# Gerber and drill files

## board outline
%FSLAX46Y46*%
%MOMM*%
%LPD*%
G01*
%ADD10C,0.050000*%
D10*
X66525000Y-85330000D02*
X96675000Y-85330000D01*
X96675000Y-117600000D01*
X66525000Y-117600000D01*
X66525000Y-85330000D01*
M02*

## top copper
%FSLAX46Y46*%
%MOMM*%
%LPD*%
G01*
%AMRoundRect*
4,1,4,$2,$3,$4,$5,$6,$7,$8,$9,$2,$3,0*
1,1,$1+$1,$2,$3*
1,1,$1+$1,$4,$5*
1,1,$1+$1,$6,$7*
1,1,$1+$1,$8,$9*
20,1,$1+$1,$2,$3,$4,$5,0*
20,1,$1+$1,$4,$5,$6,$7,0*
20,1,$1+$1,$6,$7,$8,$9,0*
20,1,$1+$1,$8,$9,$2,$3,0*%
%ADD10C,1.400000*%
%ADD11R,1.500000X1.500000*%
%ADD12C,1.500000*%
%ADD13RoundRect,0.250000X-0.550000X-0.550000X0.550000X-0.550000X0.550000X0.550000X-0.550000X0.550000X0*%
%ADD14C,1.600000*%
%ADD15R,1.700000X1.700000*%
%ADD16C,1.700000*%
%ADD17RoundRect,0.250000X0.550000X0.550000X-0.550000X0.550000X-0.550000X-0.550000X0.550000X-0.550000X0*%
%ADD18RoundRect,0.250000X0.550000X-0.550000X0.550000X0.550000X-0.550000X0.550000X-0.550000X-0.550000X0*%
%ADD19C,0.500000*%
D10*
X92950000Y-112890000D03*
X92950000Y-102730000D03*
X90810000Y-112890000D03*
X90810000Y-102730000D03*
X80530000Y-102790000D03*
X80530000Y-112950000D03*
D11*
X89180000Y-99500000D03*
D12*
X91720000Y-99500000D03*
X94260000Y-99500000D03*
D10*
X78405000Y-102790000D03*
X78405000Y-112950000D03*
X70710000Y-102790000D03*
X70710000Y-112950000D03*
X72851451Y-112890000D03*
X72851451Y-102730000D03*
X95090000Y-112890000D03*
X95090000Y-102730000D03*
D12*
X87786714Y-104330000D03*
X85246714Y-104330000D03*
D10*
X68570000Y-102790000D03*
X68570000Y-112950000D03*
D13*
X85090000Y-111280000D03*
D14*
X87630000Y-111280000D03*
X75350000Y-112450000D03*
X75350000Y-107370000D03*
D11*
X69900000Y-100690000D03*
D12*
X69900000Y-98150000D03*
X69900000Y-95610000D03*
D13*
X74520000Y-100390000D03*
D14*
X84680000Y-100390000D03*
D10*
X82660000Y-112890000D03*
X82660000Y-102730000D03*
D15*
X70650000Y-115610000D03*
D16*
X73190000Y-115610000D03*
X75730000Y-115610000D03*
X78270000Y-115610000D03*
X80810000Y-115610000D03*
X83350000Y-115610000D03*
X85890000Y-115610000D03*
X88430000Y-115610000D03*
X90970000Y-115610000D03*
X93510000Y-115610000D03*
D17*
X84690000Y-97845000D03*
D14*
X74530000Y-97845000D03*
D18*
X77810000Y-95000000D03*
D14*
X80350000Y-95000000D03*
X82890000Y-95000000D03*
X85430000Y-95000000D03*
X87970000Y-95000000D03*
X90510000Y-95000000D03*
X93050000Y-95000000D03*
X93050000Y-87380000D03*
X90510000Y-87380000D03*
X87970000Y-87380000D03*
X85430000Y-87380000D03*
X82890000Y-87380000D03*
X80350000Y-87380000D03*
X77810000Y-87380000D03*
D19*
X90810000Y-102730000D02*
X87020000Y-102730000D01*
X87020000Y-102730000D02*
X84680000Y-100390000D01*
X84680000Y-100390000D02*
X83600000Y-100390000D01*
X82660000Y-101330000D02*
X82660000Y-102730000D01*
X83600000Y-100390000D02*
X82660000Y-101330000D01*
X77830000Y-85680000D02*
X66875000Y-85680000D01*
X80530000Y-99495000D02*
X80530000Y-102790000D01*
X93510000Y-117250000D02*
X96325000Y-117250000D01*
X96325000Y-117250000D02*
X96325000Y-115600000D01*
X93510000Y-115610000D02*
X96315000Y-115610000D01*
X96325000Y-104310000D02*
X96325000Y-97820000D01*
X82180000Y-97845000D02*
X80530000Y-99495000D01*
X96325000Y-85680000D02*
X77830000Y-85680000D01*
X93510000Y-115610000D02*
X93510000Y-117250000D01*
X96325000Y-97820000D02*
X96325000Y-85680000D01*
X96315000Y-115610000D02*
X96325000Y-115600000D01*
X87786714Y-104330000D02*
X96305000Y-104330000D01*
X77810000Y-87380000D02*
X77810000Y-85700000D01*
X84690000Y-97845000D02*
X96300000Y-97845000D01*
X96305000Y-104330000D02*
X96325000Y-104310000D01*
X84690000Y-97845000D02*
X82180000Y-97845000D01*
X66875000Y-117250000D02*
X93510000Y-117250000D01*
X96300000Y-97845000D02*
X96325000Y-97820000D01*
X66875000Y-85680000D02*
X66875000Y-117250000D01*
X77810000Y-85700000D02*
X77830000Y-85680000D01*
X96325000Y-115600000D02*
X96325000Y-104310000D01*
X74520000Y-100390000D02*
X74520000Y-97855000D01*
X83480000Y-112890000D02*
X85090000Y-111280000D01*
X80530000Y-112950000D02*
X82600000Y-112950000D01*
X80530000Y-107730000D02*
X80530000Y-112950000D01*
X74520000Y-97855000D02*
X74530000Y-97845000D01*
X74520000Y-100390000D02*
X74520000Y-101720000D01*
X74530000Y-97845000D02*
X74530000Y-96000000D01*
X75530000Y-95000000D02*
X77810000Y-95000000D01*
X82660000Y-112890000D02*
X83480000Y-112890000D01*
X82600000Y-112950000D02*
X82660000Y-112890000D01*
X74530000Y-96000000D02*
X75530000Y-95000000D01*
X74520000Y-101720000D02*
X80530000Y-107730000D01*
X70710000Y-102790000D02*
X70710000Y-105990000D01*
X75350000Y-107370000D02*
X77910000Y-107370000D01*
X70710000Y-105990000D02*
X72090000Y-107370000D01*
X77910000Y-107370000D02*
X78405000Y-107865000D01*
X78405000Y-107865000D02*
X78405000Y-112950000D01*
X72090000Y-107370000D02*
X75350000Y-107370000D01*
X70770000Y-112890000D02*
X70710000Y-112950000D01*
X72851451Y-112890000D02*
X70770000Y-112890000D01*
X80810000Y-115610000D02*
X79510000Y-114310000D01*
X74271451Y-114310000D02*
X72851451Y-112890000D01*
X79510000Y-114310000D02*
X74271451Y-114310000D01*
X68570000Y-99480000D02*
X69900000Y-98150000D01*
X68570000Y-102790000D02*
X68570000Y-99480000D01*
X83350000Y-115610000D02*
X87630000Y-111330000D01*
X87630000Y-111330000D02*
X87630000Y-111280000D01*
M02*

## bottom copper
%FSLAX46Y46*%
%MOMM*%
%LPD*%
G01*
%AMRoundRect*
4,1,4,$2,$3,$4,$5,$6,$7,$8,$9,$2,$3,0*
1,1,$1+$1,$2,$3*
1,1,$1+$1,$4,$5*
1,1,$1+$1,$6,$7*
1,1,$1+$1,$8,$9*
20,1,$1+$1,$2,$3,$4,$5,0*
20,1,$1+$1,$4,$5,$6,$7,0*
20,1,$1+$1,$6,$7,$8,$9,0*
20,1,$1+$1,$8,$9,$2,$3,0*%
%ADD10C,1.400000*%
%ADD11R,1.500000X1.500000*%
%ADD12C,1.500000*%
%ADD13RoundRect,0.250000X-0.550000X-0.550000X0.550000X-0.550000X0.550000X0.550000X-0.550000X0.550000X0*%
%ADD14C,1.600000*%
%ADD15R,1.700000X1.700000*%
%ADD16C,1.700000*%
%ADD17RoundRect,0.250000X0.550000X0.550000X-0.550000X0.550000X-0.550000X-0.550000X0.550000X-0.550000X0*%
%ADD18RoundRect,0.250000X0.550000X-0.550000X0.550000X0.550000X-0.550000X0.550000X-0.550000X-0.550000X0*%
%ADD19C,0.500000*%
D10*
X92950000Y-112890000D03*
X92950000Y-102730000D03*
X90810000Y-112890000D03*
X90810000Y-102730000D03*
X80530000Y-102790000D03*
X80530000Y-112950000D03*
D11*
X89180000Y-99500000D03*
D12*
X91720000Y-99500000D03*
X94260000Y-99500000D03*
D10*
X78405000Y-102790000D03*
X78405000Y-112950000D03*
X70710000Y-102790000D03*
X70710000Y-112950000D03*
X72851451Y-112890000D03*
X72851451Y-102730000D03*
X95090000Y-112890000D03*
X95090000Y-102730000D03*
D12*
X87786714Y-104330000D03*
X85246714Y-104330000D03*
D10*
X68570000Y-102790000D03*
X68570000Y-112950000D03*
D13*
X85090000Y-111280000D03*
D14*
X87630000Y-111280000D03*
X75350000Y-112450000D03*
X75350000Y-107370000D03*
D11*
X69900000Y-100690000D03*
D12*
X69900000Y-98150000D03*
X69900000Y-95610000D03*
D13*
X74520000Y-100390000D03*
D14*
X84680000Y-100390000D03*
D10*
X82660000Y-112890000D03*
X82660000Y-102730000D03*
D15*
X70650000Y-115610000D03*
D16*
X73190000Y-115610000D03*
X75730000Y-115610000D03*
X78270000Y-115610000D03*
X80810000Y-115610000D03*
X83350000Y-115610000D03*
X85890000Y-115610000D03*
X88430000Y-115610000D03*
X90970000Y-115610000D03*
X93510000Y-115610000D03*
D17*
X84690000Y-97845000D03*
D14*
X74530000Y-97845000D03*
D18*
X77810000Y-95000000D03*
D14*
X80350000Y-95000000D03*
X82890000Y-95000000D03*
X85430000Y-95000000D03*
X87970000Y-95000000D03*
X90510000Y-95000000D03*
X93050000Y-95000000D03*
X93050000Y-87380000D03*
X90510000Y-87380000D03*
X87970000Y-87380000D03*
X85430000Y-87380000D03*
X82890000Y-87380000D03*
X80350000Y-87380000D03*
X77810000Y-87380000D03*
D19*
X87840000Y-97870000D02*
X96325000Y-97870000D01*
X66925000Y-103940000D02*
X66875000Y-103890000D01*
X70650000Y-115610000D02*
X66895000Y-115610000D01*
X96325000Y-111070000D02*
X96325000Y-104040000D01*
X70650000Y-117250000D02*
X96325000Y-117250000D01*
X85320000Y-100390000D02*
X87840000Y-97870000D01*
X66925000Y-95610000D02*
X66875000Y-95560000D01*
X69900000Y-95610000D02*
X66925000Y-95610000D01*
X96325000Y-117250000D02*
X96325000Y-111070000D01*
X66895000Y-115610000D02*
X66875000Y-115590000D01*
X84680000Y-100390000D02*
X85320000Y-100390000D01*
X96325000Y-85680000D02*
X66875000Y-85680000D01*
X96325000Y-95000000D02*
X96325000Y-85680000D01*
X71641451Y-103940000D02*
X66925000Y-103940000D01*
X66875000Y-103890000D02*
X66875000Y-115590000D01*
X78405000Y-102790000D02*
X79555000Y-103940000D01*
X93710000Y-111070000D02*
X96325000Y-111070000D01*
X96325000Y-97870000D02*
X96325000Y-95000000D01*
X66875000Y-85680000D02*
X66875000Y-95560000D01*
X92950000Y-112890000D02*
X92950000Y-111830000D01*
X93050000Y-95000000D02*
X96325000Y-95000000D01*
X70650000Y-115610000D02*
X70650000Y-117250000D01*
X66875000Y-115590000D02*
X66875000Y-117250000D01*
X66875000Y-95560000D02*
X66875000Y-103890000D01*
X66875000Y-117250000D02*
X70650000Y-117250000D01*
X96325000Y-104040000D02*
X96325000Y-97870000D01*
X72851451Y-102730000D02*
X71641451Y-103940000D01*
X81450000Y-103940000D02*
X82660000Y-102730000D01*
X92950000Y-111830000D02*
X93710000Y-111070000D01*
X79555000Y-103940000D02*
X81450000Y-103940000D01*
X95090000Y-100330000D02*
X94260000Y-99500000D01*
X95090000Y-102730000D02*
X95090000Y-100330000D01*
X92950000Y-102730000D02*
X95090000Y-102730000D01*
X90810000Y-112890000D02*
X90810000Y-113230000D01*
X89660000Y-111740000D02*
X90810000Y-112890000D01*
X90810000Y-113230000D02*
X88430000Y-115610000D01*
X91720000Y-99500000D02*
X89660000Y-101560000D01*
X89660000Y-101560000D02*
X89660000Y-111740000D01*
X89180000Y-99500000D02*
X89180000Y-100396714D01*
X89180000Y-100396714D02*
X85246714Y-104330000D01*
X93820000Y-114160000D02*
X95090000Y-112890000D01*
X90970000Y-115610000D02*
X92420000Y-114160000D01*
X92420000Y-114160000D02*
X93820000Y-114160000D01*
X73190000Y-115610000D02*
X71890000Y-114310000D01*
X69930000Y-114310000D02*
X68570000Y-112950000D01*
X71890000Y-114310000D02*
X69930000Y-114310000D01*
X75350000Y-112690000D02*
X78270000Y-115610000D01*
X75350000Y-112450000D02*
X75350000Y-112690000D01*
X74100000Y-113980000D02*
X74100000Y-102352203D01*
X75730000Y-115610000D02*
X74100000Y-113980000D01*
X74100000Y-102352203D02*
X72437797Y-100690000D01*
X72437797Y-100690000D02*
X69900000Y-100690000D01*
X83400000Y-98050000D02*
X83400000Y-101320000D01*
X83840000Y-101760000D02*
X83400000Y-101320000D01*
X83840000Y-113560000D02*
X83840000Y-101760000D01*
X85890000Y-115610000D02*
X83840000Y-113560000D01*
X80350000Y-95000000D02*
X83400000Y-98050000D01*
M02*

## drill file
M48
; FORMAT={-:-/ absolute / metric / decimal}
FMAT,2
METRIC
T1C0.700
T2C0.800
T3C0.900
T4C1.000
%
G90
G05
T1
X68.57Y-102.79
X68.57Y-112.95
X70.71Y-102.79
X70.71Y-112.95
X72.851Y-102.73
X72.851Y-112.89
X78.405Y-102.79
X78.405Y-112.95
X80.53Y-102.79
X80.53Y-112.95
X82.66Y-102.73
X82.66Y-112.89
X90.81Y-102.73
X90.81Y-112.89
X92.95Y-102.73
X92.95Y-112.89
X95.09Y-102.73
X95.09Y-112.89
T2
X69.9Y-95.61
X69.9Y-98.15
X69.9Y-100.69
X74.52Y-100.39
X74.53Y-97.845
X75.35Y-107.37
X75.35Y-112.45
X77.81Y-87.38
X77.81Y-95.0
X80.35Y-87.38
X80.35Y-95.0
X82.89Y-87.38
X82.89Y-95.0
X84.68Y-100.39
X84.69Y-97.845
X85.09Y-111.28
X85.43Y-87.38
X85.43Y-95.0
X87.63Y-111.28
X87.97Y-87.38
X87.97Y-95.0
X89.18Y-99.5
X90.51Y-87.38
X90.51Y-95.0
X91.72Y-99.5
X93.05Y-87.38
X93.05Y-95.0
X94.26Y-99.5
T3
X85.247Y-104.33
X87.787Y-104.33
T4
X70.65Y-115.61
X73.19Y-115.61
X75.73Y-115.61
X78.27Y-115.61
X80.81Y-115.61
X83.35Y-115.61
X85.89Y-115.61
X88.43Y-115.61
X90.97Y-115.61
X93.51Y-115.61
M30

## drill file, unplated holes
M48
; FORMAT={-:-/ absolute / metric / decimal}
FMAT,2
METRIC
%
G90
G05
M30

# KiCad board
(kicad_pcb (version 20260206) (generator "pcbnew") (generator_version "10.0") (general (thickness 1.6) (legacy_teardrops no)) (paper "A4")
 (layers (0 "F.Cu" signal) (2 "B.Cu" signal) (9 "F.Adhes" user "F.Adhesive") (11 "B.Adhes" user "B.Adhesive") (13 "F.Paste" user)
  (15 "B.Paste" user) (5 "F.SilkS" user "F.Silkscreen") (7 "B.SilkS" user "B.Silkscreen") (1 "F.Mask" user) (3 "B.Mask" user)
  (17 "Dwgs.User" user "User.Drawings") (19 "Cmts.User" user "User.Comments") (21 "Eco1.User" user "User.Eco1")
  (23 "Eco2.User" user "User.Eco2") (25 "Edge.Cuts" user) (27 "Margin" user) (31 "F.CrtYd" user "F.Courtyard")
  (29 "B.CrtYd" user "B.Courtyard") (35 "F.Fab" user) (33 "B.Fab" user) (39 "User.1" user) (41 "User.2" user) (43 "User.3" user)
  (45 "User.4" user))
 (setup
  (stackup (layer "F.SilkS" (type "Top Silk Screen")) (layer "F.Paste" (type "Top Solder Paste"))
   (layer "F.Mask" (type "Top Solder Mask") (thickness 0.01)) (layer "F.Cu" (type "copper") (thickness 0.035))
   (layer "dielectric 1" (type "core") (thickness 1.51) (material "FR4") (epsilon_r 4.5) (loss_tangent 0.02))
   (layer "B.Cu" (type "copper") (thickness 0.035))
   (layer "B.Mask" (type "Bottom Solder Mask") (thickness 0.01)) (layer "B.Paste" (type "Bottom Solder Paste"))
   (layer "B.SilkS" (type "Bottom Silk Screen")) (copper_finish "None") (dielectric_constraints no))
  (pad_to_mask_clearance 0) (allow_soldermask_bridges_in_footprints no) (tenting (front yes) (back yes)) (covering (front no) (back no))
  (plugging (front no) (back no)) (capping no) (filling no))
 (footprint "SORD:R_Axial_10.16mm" (layer "F.Cu") (at 92.95 112.89 90)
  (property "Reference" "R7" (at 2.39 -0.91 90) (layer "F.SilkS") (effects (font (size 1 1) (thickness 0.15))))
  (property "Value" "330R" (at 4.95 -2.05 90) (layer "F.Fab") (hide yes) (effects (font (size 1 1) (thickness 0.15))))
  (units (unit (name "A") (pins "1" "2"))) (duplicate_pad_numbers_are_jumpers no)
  (pad "1" thru_hole circle (at 0 0 90) (size 1.4 1.4) (drill 0.7) (layers "*.Cu" "*.Mask") (remove_unused_layers no) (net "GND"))
  (pad "2" thru_hole circle (at 10.16 0 90) (size 1.4 1.4) (drill 0.7) (layers "*.Cu" "*.Mask") (remove_unused_layers no) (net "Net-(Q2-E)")))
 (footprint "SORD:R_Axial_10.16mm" (layer "F.Cu") (at 90.81 112.89 90)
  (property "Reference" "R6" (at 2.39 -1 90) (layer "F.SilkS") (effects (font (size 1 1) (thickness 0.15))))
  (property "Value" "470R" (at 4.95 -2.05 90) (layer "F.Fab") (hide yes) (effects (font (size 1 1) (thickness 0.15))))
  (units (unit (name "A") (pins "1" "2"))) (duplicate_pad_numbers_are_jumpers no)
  (pad "1" thru_hole circle (at 0 0 90) (size 1.4 1.4) (drill 0.7) (layers "*.Cu" "*.Mask") (remove_unused_layers no) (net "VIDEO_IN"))
  (pad "2" thru_hole circle (at 10.16 0 90) (size 1.4 1.4) (drill 0.7) (layers "*.Cu" "*.Mask") (remove_unused_layers no) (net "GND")))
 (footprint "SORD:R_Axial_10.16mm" (layer "F.Cu") (at 80.53 102.79 -90)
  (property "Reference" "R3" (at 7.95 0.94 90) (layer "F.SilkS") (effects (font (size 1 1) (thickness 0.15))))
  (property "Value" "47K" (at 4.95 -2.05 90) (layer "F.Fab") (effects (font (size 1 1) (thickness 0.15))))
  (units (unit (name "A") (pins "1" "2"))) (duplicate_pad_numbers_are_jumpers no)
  (pad "1" thru_hole circle (at 0 0 270) (size 1.4 1.4) (drill 0.7) (layers "*.Cu" "*.Mask") (remove_unused_layers no) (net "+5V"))
  (pad "2" thru_hole circle (at 10.16 0 270) (size 1.4 1.4) (drill 0.7) (layers "*.Cu" "*.Mask") (remove_unused_layers no)
   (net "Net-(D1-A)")))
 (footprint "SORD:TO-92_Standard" (layer "F.Cu") (at 89.18 99.5)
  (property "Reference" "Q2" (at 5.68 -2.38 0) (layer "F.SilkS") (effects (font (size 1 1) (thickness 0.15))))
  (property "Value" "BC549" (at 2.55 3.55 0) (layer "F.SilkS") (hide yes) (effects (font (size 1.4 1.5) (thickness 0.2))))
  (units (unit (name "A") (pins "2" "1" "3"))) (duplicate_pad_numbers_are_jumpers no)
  (pad "1" thru_hole rect (at 0 0) (size 1.5 1.5) (drill 0.8) (layers "*.Cu" "*.Mask") (remove_unused_layers no) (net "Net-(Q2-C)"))
  (pad "2" thru_hole circle (at 2.54 0) (size 1.5 1.5) (drill 0.8) (layers "*.Cu" "*.Mask") (remove_unused_layers no) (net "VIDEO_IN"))
  (pad "3" thru_hole circle (at 5.08 0) (size 1.5 1.5) (drill 0.8) (layers "*.Cu" "*.Mask") (remove_unused_layers no) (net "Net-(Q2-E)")))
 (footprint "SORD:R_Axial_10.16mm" (layer "F.Cu") (at 78.405 102.79 -90)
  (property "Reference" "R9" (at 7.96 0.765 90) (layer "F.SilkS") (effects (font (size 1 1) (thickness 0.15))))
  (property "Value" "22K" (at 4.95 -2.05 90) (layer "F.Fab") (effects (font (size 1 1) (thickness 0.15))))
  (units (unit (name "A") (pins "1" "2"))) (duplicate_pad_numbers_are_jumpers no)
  (pad "1" thru_hole circle (at 0 0 270) (size 1.4 1.4) (drill 0.7) (layers "*.Cu" "*.Mask") (remove_unused_layers no) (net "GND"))
  (pad "2" thru_hole circle (at 10.16 0 270) (size 1.4 1.4) (drill 0.7) (layers "*.Cu" "*.Mask") (remove_unused_layers no)
   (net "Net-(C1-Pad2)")))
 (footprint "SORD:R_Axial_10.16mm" (layer "F.Cu") (at 70.71 102.79 -90)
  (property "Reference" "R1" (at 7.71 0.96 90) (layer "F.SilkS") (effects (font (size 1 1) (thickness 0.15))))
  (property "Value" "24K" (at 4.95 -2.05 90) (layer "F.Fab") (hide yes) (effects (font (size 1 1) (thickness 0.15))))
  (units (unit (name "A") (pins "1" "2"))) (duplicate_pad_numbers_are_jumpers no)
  (pad "1" thru_hole circle (at 0 0 270) (size 1.4 1.4) (drill 0.7) (layers "*.Cu" "*.Mask") (remove_unused_layers no) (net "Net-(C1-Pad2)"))
  (pad "2" thru_hole circle (at 10.16 0 270) (size 1.4 1.4) (drill 0.7) (layers "*.Cu" "*.Mask") (remove_unused_layers no) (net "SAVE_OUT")))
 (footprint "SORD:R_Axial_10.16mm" (layer "F.Cu") (at 72.851451 112.89 90)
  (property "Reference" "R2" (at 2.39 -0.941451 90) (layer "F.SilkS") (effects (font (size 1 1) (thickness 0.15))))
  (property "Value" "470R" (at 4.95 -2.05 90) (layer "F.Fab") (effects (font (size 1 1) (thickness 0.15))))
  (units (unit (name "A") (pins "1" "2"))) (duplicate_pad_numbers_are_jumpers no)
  (pad "1" thru_hole circle (at 0 0 90) (size 1.4 1.4) (drill 0.7) (layers "*.Cu" "*.Mask") (remove_unused_layers no) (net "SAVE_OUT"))
  (pad "2" thru_hole circle (at 10.16 0 90) (size 1.4 1.4) (drill 0.7) (layers "*.Cu" "*.Mask") (remove_unused_layers no) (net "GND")))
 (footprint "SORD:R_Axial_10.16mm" (layer "F.Cu") (at 95.09 112.89 90)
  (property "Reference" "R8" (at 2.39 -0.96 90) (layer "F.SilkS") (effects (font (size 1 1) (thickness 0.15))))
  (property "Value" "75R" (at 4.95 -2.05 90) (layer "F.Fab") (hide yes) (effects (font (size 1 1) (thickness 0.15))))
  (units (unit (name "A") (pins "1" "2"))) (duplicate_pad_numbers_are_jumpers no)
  (pad "1" thru_hole circle (at 0 0 90) (size 1.4 1.4) (drill 0.7) (layers "*.Cu" "*.Mask") (remove_unused_layers no) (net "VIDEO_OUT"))
  (pad "2" thru_hole circle (at 10.16 0 90) (size 1.4 1.4) (drill 0.7) (layers "*.Cu" "*.Mask") (remove_unused_layers no) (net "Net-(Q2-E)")))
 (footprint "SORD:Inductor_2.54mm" (layer "F.Cu") (at 87.786714 104.33 180)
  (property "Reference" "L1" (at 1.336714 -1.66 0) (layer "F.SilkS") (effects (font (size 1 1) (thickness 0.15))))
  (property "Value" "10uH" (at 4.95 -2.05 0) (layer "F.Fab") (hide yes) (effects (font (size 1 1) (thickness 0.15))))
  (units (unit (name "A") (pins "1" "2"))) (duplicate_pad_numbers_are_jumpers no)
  (pad "1" thru_hole circle (at 0 0 180) (size 1.5 1.5) (drill 0.9) (layers "*.Cu" "*.Mask") (remove_unused_layers no) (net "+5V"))
  (pad "2" thru_hole circle (at 2.54 0 180) (size 1.5 1.5) (drill 0.9) (layers "*.Cu" "*.Mask") (remove_unused_layers no) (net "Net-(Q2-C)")))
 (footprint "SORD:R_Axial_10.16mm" (layer "F.Cu") (at 68.57 102.79 -90)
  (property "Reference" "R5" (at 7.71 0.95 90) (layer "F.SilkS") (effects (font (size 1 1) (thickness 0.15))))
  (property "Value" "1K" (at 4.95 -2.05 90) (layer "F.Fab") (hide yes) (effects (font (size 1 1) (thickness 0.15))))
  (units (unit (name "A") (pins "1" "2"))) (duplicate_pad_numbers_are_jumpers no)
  (pad "1" thru_hole circle (at 0 0 270) (size 1.4 1.4) (drill 0.7) (layers "*.Cu" "*.Mask") (remove_unused_layers no) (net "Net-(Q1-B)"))
  (pad "2" thru_hole circle (at 10.16 0 270) (size 1.4 1.4) (drill 0.7) (layers "*.Cu" "*.Mask") (remove_unused_layers no) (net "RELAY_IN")))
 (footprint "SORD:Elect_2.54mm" (layer "F.Cu") (at 85.09 111.28)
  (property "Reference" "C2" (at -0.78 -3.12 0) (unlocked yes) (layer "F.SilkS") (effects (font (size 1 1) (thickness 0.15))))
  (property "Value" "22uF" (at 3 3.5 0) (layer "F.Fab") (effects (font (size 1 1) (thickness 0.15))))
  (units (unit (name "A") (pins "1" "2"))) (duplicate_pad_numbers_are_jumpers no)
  (pad "1" thru_hole roundrect (at 0 0) (size 1.6 1.6) (drill 0.8) (layers "*.Cu" "*.Mask") (remove_unused_layers no)
   (roundrect_rratio 0.15625) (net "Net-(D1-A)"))
  (pad "2" thru_hole circle (at 2.54 0) (size 1.6 1.6) (drill 0.8) (layers "*.Cu" "*.Mask") (remove_unused_layers no) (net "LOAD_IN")))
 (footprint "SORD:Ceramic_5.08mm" (layer "F.Cu") (at 75.35 112.45 90)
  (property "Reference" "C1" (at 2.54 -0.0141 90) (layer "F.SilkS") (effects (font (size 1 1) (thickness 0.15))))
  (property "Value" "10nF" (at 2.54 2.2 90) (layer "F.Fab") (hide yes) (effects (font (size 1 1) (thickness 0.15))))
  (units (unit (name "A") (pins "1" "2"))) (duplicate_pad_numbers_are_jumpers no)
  (pad "1" thru_hole circle (at 0 0 90) (size 1.6 1.6) (drill 0.8) (layers "*.Cu" "*.Mask") (remove_unused_layers no) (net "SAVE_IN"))
  (pad "2" thru_hole circle (at 5.08 0 90) (size 1.6 1.6) (drill 0.8) (layers "*.Cu" "*.Mask") (remove_unused_layers no)
   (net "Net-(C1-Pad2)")))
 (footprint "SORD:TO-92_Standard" (layer "F.Cu") (at 69.9 100.69 90)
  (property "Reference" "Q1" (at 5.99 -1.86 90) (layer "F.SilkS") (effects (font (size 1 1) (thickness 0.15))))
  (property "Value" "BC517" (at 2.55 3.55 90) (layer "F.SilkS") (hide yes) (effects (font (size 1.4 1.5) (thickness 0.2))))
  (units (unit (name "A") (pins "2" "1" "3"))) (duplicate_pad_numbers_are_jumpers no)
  (pad "1" thru_hole rect (at 0 0 90) (size 1.5 1.5) (drill 0.8) (layers "*.Cu" "*.Mask") (remove_unused_layers no) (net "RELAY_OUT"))
  (pad "2" thru_hole circle (at 2.54 0 90) (size 1.5 1.5) (drill 0.8) (layers "*.Cu" "*.Mask") (remove_unused_layers no) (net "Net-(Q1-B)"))
  (pad "3" thru_hole circle (at 5.08 0 90) (size 1.5 1.5) (drill 0.8) (layers "*.Cu" "*.Mask") (remove_unused_layers no) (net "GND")))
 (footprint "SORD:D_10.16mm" (layer "F.Cu") (at 74.52 100.39)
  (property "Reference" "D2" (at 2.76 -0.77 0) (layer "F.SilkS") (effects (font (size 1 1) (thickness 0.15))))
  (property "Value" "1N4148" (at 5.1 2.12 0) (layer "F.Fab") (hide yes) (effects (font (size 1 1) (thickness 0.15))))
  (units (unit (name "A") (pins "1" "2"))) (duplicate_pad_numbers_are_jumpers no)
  (pad "1" thru_hole roundrect (at 0 0) (size 1.6 1.6) (drill 0.8) (layers "*.Cu" "*.Mask") (remove_unused_layers no)
   (roundrect_rratio 0.15625) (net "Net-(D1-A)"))
  (pad "2" thru_hole circle (at 10.16 0) (size 1.6 1.6) (drill 0.8) (layers "*.Cu" "*.Mask") (remove_unused_layers no) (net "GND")))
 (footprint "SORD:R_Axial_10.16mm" (layer "F.Cu") (at 82.66 112.89 90)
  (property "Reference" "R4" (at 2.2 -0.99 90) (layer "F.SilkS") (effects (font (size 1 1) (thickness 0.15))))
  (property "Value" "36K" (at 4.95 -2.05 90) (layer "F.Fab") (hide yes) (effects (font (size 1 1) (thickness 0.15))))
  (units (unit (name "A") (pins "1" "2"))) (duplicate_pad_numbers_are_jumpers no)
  (pad "1" thru_hole circle (at 0 0 90) (size 1.4 1.4) (drill 0.7) (layers "*.Cu" "*.Mask") (remove_unused_layers no) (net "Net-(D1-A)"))
  (pad "2" thru_hole circle (at 10.16 0 90) (size 1.4 1.4) (drill 0.7) (layers "*.Cu" "*.Mask") (remove_unused_layers no) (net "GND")))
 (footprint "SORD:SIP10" (layer "F.Cu") (at 70.65 115.61)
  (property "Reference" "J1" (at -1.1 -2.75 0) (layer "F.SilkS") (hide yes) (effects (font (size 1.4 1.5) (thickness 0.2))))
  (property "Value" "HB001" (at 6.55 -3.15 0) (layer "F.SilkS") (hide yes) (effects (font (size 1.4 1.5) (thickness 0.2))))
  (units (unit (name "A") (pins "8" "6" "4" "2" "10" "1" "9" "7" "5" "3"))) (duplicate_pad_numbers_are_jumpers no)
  (pad "1" thru_hole rect (at 0 0) (size 1.7 1.7) (drill 1) (layers "*.Cu" "*.Mask") (remove_unused_layers no) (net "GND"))
  (pad "2" thru_hole circle (at 2.54 0) (size 1.7 1.7) (drill 1) (layers "*.Cu" "*.Mask") (remove_unused_layers no) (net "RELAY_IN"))
  (pad "3" thru_hole circle (at 5.08 0) (size 1.7 1.7) (drill 1) (layers "*.Cu" "*.Mask") (remove_unused_layers no) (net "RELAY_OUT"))
  (pad "4" thru_hole circle (at 7.62 0) (size 1.7 1.7) (drill 1) (layers "*.Cu" "*.Mask") (remove_unused_layers no) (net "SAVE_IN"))
  (pad "5" thru_hole circle (at 10.16 0) (size 1.7 1.7) (drill 1) (layers "*.Cu" "*.Mask") (remove_unused_layers no) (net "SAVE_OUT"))
  (pad "6" thru_hole circle (at 12.7 0) (size 1.7 1.7) (drill 1) (layers "*.Cu" "*.Mask") (remove_unused_layers no) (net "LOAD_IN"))
  (pad "7" thru_hole circle (at 15.24 0) (size 1.7 1.7) (drill 1) (layers "*.Cu" "*.Mask") (remove_unused_layers no) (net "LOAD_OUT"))
  (pad "8" thru_hole circle (at 17.78 0) (size 1.7 1.7) (drill 1) (layers "*.Cu" "*.Mask") (remove_unused_layers no) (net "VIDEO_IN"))
  (pad "9" thru_hole circle (at 20.32 0) (size 1.7 1.7) (drill 1) (layers "*.Cu" "*.Mask") (remove_unused_layers no) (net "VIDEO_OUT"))
  (pad "10" thru_hole circle (at 22.86 0) (size 1.7 1.7) (drill 1) (layers "*.Cu" "*.Mask") (remove_unused_layers no) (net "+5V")))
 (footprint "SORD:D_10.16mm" (layer "F.Cu") (at 84.69 97.845 180)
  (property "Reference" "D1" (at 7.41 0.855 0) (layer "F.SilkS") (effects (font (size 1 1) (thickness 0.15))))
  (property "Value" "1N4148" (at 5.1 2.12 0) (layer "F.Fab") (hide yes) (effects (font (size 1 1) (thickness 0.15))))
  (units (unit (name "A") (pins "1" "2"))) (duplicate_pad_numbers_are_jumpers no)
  (pad "1" thru_hole roundrect (at 0 0 180) (size 1.6 1.6) (drill 0.8) (layers "*.Cu" "*.Mask") (remove_unused_layers no)
   (roundrect_rratio 0.15625) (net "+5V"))
  (pad "2" thru_hole circle (at 10.16 0 180) (size 1.6 1.6) (drill 0.8) (layers "*.Cu" "*.Mask") (remove_unused_layers no)
   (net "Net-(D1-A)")))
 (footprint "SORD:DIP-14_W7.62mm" (layer "F.Cu") (at 77.81 95 90)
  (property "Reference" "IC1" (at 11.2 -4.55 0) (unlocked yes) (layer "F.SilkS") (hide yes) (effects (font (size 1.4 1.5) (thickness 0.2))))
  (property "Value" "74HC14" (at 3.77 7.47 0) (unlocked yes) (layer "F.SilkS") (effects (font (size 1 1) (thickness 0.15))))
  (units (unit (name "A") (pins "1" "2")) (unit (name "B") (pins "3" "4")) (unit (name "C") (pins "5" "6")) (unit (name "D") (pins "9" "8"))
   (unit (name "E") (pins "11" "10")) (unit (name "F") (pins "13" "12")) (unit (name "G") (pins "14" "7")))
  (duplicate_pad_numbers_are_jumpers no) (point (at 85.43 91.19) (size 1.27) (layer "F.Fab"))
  (pad "1" thru_hole roundrect (at 0 0 90) (size 1.6 1.6) (drill 0.8) (layers "*.Cu" "*.Mask") (remove_unused_layers no)
   (roundrect_rratio 0.15625) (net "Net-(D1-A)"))
  (pad "2" thru_hole circle (at 0 2.54 90) (size 1.6 1.6) (drill 0.8) (layers "*.Cu" "*.Mask") (remove_unused_layers no) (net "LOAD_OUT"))
  (pad "3" thru_hole circle (at 0 5.08 90) (size 1.6 1.6) (drill 0.8) (layers "*.Cu" "*.Mask") (remove_unused_layers no)
   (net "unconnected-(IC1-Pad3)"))
  (pad "4" thru_hole circle (at 0 7.62 90) (size 1.6 1.6) (drill 0.8) (layers "*.Cu" "*.Mask") (remove_unused_layers no)
   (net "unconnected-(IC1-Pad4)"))
  (pad "5" thru_hole circle (at 0 10.16 90) (size 1.6 1.6) (drill 0.8) (layers "*.Cu" "*.Mask") (remove_unused_layers no)
   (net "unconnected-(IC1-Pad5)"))
  (pad "6" thru_hole circle (at 0 12.7 90) (size 1.6 1.6) (drill 0.8) (layers "*.Cu" "*.Mask") (remove_unused_layers no)
   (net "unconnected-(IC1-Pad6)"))
  (pad "7" thru_hole circle (at 0 15.24 90) (size 1.6 1.6) (drill 0.8) (layers "*.Cu" "*.Mask") (remove_unused_layers no) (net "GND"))
  (pad "8" thru_hole circle (at 7.62 15.24 90) (size 1.6 1.6) (drill 0.8) (layers "*.Cu" "*.Mask") (remove_unused_layers no)
   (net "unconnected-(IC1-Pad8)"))
  (pad "9" thru_hole circle (at 7.62 12.7 90) (size 1.6 1.6) (drill 0.8) (layers "*.Cu" "*.Mask") (remove_unused_layers no)
   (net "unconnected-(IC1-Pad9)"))
  (pad "10" thru_hole circle (at 7.62 10.16 90) (size 1.6 1.6) (drill 0.8) (layers "*.Cu" "*.Mask") (remove_unused_layers no)
   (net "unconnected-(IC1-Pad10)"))
  (pad "11" thru_hole circle (at 7.62 7.62 90) (size 1.6 1.6) (drill 0.8) (layers "*.Cu" "*.Mask") (remove_unused_layers no)
   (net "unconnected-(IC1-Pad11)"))
  (pad "12" thru_hole circle (at 7.62 5.08 90) (size 1.6 1.6) (drill 0.8) (layers "*.Cu" "*.Mask") (remove_unused_layers no)
   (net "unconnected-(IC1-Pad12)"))
  (pad "13" thru_hole circle (at 7.62 2.54 90) (size 1.6 1.6) (drill 0.8) (layers "*.Cu" "*.Mask") (remove_unused_layers no)
   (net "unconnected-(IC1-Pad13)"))
  (pad "14" thru_hole circle (at 7.62 0 90) (size 1.6 1.6) (drill 0.8) (layers "*.Cu" "*.Mask") (remove_unused_layers no) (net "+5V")))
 (gr_rect (start 66.525 85.33) (end 96.675 117.6) (stroke (width 0.05) (type default)) (fill no) (layer "Edge.Cuts"))
 (segment (start 90.81 102.73) (end 87.02 102.73) (width 0.5) (layer "F.Cu") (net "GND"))
 (segment (start 87.02 102.73) (end 84.68 100.39) (width 0.5) (layer "F.Cu") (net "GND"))
 (segment (start 84.68 100.39) (end 83.6 100.39) (width 0.5) (layer "F.Cu") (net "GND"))
 (segment (start 82.66 101.33) (end 82.66 102.73) (width 0.5) (layer "F.Cu") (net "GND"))
 (segment (start 83.6 100.39) (end 82.66 101.33) (width 0.5) (layer "F.Cu") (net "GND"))
 (segment (start 87.84 97.87) (end 96.325 97.87) (width 0.5) (layer "B.Cu") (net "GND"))
 (segment (start 66.925 103.94) (end 66.875 103.89) (width 0.5) (layer "B.Cu") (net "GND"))
 (segment (start 70.65 115.61) (end 66.895 115.61) (width 0.5) (layer "B.Cu") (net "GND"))
 (segment (start 96.325 111.07) (end 96.325 104.04) (width 0.5) (layer "B.Cu") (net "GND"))
 (segment (start 70.65 117.25) (end 96.325 117.25) (width 0.5) (layer "B.Cu") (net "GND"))
 (segment (start 85.32 100.39) (end 87.84 97.87) (width 0.5) (layer "B.Cu") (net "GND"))
 (segment (start 66.925 95.61) (end 66.875 95.56) (width 0.5) (layer "B.Cu") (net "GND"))
 (segment (start 69.9 95.61) (end 66.925 95.61) (width 0.5) (layer "B.Cu") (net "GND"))
 (segment (start 96.325 117.25) (end 96.325 111.07) (width 0.5) (layer "B.Cu") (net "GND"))
 (segment (start 66.895 115.61) (end 66.875 115.59) (width 0.5) (layer "B.Cu") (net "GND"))
 (segment (start 84.68 100.39) (end 85.32 100.39) (width 0.5) (layer "B.Cu") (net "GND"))
 (segment (start 96.325 85.68) (end 66.875 85.68) (width 0.5) (layer "B.Cu") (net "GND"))
 (segment (start 96.325 95) (end 96.325 85.68) (width 0.5) (layer "B.Cu") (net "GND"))
 (segment (start 71.641451 103.94) (end 66.925 103.94) (width 0.5) (layer "B.Cu") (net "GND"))
 (segment (start 66.875 103.89) (end 66.875 115.59) (width 0.5) (layer "B.Cu") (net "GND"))
 (segment (start 78.405 102.79) (end 79.555 103.94) (width 0.5) (layer "B.Cu") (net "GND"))
 (segment (start 93.71 111.07) (end 96.325 111.07) (width 0.5) (layer "B.Cu") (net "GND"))
 (segment (start 96.325 97.87) (end 96.325 95) (width 0.5) (layer "B.Cu") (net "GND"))
 (segment (start 66.875 85.68) (end 66.875 95.56) (width 0.5) (layer "B.Cu") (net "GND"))
 (segment (start 92.95 112.89) (end 92.95 111.83) (width 0.5) (layer "B.Cu") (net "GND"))
 (segment (start 93.05 95) (end 96.325 95) (width 0.5) (layer "B.Cu") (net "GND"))
 (segment (start 70.65 115.61) (end 70.65 117.25) (width 0.5) (layer "B.Cu") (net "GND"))
 (segment (start 66.875 115.59) (end 66.875 117.25) (width 0.5) (layer "B.Cu") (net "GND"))
 (segment (start 66.875 95.56) (end 66.875 103.89) (width 0.5) (layer "B.Cu") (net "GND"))
 (segment (start 66.875 117.25) (end 70.65 117.25) (width 0.5) (layer "B.Cu") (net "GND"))
 (segment (start 96.325 104.04) (end 96.325 97.87) (width 0.5) (layer "B.Cu") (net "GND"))
 (segment (start 72.851451 102.73) (end 71.641451 103.94) (width 0.5) (layer "B.Cu") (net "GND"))
 (segment (start 81.45 103.94) (end 82.66 102.73) (width 0.5) (layer "B.Cu") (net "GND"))
 (segment (start 92.95 111.83) (end 93.71 111.07) (width 0.5) (layer "B.Cu") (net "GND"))
 (segment (start 79.555 103.94) (end 81.45 103.94) (width 0.5) (layer "B.Cu") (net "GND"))
 (segment (start 95.09 100.33) (end 94.26 99.5) (width 0.5) (layer "B.Cu") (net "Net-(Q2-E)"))
 (segment (start 95.09 102.73) (end 95.09 100.33) (width 0.5) (layer "B.Cu") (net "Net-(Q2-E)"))
 (segment (start 92.95 102.73) (end 95.09 102.73) (width 0.5) (layer "B.Cu") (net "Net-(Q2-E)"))
 (segment (start 90.81 112.89) (end 90.81 113.23) (width 0.5) (layer "B.Cu") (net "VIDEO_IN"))
 (segment (start 89.66 111.74) (end 90.81 112.89) (width 0.5) (layer "B.Cu") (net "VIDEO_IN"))
 (segment (start 90.81 113.23) (end 88.43 115.61) (width 0.5) (layer "B.Cu") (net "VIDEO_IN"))
 (segment (start 91.72 99.5) (end 89.66 101.56) (width 0.5) (layer "B.Cu") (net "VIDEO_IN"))
 (segment (start 89.66 101.56) (end 89.66 111.74) (width 0.5) (layer "B.Cu") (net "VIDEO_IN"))
 (segment (start 77.83 85.68) (end 66.875 85.68) (width 0.5) (layer "F.Cu") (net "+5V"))
 (segment (start 80.53 99.495) (end 80.53 102.79) (width 0.5) (layer "F.Cu") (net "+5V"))
 (segment (start 93.51 117.25) (end 96.325 117.25) (width 0.5) (layer "F.Cu") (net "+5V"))
 (segment (start 96.325 117.25) (end 96.325 115.6) (width 0.5) (layer "F.Cu") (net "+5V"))
 (segment (start 93.51 115.61) (end 96.315 115.61) (width 0.5) (layer "F.Cu") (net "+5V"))
 (segment (start 96.325 104.31) (end 96.325 97.82) (width 0.5) (layer "F.Cu") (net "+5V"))
 (segment (start 82.18 97.845) (end 80.53 99.495) (width 0.5) (layer "F.Cu") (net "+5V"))
 (segment (start 96.325 85.68) (end 77.83 85.68) (width 0.5) (layer "F.Cu") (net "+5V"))
 (segment (start 93.51 115.61) (end 93.51 117.25) (width 0.5) (layer "F.Cu") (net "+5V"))
 (segment (start 96.325 97.82) (end 96.325 85.68) (width 0.5) (layer "F.Cu") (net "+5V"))
 (segment (start 96.315 115.61) (end 96.325 115.6) (width 0.5) (layer "F.Cu") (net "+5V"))
 (segment (start 87.786714 104.33) (end 96.305 104.33) (width 0.5) (layer "F.Cu") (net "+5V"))
 (segment (start 77.81 87.38) (end 77.81 85.7) (width 0.5) (layer "F.Cu") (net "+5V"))
 (segment (start 84.69 97.845) (end 96.3 97.845) (width 0.5) (layer "F.Cu") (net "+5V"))
 (segment (start 96.305 104.33) (end 96.325 104.31) (width 0.5) (layer "F.Cu") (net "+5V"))
 (segment (start 84.69 97.845) (end 82.18 97.845) (width 0.5) (layer "F.Cu") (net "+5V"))
 (segment (start 66.875 117.25) (end 93.51 117.25) (width 0.5) (layer "F.Cu") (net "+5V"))
 (segment (start 96.3 97.845) (end 96.325 97.82) (width 0.5) (layer "F.Cu") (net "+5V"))
 (segment (start 66.875 85.68) (end 66.875 117.25) (width 0.5) (layer "F.Cu") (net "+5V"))
 (segment (start 77.81 85.7) (end 77.83 85.68) (width 0.5) (layer "F.Cu") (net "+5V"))
 (segment (start 96.325 115.6) (end 96.325 104.31) (width 0.5) (layer "F.Cu") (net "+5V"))
 (segment (start 74.52 100.39) (end 74.52 97.855) (width 0.5) (layer "F.Cu") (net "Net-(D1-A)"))
 (segment (start 83.48 112.89) (end 85.09 111.28) (width 0.5) (layer "F.Cu") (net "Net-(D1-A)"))
 (segment (start 80.53 112.95) (end 82.6 112.95) (width 0.5) (layer "F.Cu") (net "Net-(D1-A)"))
 (segment (start 80.53 107.73) (end 80.53 112.95) (width 0.5) (layer "F.Cu") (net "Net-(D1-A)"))
 (segment (start 74.52 97.855) (end 74.53 97.845) (width 0.5) (layer "F.Cu") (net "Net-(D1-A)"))
 (segment (start 74.52 100.39) (end 74.52 101.72) (width 0.5) (layer "F.Cu") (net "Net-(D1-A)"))
 (segment (start 74.53 97.845) (end 74.53 96) (width 0.5) (layer "F.Cu") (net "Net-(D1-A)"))
 (segment (start 75.53 95) (end 77.81 95) (width 0.5) (layer "F.Cu") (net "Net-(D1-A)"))
 (segment (start 82.66 112.89) (end 83.48 112.89) (width 0.5) (layer "F.Cu") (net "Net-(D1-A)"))
 (segment (start 82.6 112.95) (end 82.66 112.89) (width 0.5) (layer "F.Cu") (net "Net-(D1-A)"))
 (segment (start 74.53 96) (end 75.53 95) (width 0.5) (layer "F.Cu") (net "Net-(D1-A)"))
 (segment (start 74.52 101.72) (end 80.53 107.73) (width 0.5) (layer "F.Cu") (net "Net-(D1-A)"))
 (segment (start 89.18 99.5) (end 89.18 100.396714) (width 0.5) (layer "B.Cu") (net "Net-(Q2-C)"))
 (segment (start 89.18 100.396714) (end 85.246714 104.33) (width 0.5) (layer "B.Cu") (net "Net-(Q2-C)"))
 (segment (start 70.71 102.79) (end 70.71 105.99) (width 0.5) (layer "F.Cu") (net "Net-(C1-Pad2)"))
 (segment (start 75.35 107.37) (end 77.91 107.37) (width 0.5) (layer "F.Cu") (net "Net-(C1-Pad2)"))
 (segment (start 70.71 105.99) (end 72.09 107.37) (width 0.5) (layer "F.Cu") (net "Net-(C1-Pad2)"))
 (segment (start 77.91 107.37) (end 78.405 107.865) (width 0.5) (layer "F.Cu") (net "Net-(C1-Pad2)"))
 (segment (start 78.405 107.865) (end 78.405 112.95) (width 0.5) (layer "F.Cu") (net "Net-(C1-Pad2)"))
 (segment (start 72.09 107.37) (end 75.35 107.37) (width 0.5) (layer "F.Cu") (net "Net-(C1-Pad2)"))
 (segment (start 70.77 112.89) (end 70.71 112.95) (width 0.5) (layer "F.Cu") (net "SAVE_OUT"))
 (segment (start 72.851451 112.89) (end 70.77 112.89) (width 0.5) (layer "F.Cu") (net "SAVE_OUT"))
 (segment (start 80.81 115.61) (end 79.51 114.31) (width 0.5) (layer "F.Cu") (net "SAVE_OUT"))
 (segment (start 74.271451 114.31) (end 72.851451 112.89) (width 0.5) (layer "F.Cu") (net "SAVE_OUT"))
 (segment (start 79.51 114.31) (end 74.271451 114.31) (width 0.5) (layer "F.Cu") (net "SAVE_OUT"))
 (segment (start 93.82 114.16) (end 95.09 112.89) (width 0.5) (layer "B.Cu") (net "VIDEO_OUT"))
 (segment (start 90.97 115.61) (end 92.42 114.16) (width 0.5) (layer "B.Cu") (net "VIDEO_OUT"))
 (segment (start 92.42 114.16) (end 93.82 114.16) (width 0.5) (layer "B.Cu") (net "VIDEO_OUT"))
 (segment (start 68.57 99.48) (end 69.9 98.15) (width 0.5) (layer "F.Cu") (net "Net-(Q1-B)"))
 (segment (start 68.57 102.79) (end 68.57 99.48) (width 0.5) (layer "F.Cu") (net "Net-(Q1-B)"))
 (segment (start 73.19 115.61) (end 71.89 114.31) (width 0.5) (layer "B.Cu") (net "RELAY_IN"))
 (segment (start 69.93 114.31) (end 68.57 112.95) (width 0.5) (layer "B.Cu") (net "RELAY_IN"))
 (segment (start 71.89 114.31) (end 69.93 114.31) (width 0.5) (layer "B.Cu") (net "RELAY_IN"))
 (segment (start 83.35 115.61) (end 87.63 111.33) (width 0.5) (layer "F.Cu") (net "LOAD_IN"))
 (segment (start 87.63 111.33) (end 87.63 111.28) (width 0.5) (layer "F.Cu") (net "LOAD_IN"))
 (segment (start 75.35 112.69) (end 78.27 115.61) (width 0.5) (layer "B.Cu") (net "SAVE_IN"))
 (segment (start 75.35 112.45) (end 75.35 112.69) (width 0.5) (layer "B.Cu") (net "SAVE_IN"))
 (segment (start 74.1 113.98) (end 74.1 102.352203) (width 0.5) (layer "B.Cu") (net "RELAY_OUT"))
 (segment (start 75.73 115.61) (end 74.1 113.98) (width 0.5) (layer "B.Cu") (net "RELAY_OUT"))
 (segment (start 74.1 102.352203) (end 72.437797 100.69) (width 0.5) (layer "B.Cu") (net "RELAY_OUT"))
 (segment (start 72.437797 100.69) (end 69.9 100.69) (width 0.5) (layer "B.Cu") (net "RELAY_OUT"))
 (segment (start 83.4 98.05) (end 83.4 101.32) (width 0.5) (layer "B.Cu") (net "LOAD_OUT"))
 (segment (start 83.84 101.76) (end 83.4 101.32) (width 0.5) (layer "B.Cu") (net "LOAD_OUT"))
 (segment (start 83.84 113.56) (end 83.84 101.76) (width 0.5) (layer "B.Cu") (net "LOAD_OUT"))
 (segment (start 85.89 115.61) (end 83.84 113.56) (width 0.5) (layer "B.Cu") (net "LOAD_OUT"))
 (segment (start 80.35 95) (end 83.4 98.05) (width 0.5) (layer "B.Cu") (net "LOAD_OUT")))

